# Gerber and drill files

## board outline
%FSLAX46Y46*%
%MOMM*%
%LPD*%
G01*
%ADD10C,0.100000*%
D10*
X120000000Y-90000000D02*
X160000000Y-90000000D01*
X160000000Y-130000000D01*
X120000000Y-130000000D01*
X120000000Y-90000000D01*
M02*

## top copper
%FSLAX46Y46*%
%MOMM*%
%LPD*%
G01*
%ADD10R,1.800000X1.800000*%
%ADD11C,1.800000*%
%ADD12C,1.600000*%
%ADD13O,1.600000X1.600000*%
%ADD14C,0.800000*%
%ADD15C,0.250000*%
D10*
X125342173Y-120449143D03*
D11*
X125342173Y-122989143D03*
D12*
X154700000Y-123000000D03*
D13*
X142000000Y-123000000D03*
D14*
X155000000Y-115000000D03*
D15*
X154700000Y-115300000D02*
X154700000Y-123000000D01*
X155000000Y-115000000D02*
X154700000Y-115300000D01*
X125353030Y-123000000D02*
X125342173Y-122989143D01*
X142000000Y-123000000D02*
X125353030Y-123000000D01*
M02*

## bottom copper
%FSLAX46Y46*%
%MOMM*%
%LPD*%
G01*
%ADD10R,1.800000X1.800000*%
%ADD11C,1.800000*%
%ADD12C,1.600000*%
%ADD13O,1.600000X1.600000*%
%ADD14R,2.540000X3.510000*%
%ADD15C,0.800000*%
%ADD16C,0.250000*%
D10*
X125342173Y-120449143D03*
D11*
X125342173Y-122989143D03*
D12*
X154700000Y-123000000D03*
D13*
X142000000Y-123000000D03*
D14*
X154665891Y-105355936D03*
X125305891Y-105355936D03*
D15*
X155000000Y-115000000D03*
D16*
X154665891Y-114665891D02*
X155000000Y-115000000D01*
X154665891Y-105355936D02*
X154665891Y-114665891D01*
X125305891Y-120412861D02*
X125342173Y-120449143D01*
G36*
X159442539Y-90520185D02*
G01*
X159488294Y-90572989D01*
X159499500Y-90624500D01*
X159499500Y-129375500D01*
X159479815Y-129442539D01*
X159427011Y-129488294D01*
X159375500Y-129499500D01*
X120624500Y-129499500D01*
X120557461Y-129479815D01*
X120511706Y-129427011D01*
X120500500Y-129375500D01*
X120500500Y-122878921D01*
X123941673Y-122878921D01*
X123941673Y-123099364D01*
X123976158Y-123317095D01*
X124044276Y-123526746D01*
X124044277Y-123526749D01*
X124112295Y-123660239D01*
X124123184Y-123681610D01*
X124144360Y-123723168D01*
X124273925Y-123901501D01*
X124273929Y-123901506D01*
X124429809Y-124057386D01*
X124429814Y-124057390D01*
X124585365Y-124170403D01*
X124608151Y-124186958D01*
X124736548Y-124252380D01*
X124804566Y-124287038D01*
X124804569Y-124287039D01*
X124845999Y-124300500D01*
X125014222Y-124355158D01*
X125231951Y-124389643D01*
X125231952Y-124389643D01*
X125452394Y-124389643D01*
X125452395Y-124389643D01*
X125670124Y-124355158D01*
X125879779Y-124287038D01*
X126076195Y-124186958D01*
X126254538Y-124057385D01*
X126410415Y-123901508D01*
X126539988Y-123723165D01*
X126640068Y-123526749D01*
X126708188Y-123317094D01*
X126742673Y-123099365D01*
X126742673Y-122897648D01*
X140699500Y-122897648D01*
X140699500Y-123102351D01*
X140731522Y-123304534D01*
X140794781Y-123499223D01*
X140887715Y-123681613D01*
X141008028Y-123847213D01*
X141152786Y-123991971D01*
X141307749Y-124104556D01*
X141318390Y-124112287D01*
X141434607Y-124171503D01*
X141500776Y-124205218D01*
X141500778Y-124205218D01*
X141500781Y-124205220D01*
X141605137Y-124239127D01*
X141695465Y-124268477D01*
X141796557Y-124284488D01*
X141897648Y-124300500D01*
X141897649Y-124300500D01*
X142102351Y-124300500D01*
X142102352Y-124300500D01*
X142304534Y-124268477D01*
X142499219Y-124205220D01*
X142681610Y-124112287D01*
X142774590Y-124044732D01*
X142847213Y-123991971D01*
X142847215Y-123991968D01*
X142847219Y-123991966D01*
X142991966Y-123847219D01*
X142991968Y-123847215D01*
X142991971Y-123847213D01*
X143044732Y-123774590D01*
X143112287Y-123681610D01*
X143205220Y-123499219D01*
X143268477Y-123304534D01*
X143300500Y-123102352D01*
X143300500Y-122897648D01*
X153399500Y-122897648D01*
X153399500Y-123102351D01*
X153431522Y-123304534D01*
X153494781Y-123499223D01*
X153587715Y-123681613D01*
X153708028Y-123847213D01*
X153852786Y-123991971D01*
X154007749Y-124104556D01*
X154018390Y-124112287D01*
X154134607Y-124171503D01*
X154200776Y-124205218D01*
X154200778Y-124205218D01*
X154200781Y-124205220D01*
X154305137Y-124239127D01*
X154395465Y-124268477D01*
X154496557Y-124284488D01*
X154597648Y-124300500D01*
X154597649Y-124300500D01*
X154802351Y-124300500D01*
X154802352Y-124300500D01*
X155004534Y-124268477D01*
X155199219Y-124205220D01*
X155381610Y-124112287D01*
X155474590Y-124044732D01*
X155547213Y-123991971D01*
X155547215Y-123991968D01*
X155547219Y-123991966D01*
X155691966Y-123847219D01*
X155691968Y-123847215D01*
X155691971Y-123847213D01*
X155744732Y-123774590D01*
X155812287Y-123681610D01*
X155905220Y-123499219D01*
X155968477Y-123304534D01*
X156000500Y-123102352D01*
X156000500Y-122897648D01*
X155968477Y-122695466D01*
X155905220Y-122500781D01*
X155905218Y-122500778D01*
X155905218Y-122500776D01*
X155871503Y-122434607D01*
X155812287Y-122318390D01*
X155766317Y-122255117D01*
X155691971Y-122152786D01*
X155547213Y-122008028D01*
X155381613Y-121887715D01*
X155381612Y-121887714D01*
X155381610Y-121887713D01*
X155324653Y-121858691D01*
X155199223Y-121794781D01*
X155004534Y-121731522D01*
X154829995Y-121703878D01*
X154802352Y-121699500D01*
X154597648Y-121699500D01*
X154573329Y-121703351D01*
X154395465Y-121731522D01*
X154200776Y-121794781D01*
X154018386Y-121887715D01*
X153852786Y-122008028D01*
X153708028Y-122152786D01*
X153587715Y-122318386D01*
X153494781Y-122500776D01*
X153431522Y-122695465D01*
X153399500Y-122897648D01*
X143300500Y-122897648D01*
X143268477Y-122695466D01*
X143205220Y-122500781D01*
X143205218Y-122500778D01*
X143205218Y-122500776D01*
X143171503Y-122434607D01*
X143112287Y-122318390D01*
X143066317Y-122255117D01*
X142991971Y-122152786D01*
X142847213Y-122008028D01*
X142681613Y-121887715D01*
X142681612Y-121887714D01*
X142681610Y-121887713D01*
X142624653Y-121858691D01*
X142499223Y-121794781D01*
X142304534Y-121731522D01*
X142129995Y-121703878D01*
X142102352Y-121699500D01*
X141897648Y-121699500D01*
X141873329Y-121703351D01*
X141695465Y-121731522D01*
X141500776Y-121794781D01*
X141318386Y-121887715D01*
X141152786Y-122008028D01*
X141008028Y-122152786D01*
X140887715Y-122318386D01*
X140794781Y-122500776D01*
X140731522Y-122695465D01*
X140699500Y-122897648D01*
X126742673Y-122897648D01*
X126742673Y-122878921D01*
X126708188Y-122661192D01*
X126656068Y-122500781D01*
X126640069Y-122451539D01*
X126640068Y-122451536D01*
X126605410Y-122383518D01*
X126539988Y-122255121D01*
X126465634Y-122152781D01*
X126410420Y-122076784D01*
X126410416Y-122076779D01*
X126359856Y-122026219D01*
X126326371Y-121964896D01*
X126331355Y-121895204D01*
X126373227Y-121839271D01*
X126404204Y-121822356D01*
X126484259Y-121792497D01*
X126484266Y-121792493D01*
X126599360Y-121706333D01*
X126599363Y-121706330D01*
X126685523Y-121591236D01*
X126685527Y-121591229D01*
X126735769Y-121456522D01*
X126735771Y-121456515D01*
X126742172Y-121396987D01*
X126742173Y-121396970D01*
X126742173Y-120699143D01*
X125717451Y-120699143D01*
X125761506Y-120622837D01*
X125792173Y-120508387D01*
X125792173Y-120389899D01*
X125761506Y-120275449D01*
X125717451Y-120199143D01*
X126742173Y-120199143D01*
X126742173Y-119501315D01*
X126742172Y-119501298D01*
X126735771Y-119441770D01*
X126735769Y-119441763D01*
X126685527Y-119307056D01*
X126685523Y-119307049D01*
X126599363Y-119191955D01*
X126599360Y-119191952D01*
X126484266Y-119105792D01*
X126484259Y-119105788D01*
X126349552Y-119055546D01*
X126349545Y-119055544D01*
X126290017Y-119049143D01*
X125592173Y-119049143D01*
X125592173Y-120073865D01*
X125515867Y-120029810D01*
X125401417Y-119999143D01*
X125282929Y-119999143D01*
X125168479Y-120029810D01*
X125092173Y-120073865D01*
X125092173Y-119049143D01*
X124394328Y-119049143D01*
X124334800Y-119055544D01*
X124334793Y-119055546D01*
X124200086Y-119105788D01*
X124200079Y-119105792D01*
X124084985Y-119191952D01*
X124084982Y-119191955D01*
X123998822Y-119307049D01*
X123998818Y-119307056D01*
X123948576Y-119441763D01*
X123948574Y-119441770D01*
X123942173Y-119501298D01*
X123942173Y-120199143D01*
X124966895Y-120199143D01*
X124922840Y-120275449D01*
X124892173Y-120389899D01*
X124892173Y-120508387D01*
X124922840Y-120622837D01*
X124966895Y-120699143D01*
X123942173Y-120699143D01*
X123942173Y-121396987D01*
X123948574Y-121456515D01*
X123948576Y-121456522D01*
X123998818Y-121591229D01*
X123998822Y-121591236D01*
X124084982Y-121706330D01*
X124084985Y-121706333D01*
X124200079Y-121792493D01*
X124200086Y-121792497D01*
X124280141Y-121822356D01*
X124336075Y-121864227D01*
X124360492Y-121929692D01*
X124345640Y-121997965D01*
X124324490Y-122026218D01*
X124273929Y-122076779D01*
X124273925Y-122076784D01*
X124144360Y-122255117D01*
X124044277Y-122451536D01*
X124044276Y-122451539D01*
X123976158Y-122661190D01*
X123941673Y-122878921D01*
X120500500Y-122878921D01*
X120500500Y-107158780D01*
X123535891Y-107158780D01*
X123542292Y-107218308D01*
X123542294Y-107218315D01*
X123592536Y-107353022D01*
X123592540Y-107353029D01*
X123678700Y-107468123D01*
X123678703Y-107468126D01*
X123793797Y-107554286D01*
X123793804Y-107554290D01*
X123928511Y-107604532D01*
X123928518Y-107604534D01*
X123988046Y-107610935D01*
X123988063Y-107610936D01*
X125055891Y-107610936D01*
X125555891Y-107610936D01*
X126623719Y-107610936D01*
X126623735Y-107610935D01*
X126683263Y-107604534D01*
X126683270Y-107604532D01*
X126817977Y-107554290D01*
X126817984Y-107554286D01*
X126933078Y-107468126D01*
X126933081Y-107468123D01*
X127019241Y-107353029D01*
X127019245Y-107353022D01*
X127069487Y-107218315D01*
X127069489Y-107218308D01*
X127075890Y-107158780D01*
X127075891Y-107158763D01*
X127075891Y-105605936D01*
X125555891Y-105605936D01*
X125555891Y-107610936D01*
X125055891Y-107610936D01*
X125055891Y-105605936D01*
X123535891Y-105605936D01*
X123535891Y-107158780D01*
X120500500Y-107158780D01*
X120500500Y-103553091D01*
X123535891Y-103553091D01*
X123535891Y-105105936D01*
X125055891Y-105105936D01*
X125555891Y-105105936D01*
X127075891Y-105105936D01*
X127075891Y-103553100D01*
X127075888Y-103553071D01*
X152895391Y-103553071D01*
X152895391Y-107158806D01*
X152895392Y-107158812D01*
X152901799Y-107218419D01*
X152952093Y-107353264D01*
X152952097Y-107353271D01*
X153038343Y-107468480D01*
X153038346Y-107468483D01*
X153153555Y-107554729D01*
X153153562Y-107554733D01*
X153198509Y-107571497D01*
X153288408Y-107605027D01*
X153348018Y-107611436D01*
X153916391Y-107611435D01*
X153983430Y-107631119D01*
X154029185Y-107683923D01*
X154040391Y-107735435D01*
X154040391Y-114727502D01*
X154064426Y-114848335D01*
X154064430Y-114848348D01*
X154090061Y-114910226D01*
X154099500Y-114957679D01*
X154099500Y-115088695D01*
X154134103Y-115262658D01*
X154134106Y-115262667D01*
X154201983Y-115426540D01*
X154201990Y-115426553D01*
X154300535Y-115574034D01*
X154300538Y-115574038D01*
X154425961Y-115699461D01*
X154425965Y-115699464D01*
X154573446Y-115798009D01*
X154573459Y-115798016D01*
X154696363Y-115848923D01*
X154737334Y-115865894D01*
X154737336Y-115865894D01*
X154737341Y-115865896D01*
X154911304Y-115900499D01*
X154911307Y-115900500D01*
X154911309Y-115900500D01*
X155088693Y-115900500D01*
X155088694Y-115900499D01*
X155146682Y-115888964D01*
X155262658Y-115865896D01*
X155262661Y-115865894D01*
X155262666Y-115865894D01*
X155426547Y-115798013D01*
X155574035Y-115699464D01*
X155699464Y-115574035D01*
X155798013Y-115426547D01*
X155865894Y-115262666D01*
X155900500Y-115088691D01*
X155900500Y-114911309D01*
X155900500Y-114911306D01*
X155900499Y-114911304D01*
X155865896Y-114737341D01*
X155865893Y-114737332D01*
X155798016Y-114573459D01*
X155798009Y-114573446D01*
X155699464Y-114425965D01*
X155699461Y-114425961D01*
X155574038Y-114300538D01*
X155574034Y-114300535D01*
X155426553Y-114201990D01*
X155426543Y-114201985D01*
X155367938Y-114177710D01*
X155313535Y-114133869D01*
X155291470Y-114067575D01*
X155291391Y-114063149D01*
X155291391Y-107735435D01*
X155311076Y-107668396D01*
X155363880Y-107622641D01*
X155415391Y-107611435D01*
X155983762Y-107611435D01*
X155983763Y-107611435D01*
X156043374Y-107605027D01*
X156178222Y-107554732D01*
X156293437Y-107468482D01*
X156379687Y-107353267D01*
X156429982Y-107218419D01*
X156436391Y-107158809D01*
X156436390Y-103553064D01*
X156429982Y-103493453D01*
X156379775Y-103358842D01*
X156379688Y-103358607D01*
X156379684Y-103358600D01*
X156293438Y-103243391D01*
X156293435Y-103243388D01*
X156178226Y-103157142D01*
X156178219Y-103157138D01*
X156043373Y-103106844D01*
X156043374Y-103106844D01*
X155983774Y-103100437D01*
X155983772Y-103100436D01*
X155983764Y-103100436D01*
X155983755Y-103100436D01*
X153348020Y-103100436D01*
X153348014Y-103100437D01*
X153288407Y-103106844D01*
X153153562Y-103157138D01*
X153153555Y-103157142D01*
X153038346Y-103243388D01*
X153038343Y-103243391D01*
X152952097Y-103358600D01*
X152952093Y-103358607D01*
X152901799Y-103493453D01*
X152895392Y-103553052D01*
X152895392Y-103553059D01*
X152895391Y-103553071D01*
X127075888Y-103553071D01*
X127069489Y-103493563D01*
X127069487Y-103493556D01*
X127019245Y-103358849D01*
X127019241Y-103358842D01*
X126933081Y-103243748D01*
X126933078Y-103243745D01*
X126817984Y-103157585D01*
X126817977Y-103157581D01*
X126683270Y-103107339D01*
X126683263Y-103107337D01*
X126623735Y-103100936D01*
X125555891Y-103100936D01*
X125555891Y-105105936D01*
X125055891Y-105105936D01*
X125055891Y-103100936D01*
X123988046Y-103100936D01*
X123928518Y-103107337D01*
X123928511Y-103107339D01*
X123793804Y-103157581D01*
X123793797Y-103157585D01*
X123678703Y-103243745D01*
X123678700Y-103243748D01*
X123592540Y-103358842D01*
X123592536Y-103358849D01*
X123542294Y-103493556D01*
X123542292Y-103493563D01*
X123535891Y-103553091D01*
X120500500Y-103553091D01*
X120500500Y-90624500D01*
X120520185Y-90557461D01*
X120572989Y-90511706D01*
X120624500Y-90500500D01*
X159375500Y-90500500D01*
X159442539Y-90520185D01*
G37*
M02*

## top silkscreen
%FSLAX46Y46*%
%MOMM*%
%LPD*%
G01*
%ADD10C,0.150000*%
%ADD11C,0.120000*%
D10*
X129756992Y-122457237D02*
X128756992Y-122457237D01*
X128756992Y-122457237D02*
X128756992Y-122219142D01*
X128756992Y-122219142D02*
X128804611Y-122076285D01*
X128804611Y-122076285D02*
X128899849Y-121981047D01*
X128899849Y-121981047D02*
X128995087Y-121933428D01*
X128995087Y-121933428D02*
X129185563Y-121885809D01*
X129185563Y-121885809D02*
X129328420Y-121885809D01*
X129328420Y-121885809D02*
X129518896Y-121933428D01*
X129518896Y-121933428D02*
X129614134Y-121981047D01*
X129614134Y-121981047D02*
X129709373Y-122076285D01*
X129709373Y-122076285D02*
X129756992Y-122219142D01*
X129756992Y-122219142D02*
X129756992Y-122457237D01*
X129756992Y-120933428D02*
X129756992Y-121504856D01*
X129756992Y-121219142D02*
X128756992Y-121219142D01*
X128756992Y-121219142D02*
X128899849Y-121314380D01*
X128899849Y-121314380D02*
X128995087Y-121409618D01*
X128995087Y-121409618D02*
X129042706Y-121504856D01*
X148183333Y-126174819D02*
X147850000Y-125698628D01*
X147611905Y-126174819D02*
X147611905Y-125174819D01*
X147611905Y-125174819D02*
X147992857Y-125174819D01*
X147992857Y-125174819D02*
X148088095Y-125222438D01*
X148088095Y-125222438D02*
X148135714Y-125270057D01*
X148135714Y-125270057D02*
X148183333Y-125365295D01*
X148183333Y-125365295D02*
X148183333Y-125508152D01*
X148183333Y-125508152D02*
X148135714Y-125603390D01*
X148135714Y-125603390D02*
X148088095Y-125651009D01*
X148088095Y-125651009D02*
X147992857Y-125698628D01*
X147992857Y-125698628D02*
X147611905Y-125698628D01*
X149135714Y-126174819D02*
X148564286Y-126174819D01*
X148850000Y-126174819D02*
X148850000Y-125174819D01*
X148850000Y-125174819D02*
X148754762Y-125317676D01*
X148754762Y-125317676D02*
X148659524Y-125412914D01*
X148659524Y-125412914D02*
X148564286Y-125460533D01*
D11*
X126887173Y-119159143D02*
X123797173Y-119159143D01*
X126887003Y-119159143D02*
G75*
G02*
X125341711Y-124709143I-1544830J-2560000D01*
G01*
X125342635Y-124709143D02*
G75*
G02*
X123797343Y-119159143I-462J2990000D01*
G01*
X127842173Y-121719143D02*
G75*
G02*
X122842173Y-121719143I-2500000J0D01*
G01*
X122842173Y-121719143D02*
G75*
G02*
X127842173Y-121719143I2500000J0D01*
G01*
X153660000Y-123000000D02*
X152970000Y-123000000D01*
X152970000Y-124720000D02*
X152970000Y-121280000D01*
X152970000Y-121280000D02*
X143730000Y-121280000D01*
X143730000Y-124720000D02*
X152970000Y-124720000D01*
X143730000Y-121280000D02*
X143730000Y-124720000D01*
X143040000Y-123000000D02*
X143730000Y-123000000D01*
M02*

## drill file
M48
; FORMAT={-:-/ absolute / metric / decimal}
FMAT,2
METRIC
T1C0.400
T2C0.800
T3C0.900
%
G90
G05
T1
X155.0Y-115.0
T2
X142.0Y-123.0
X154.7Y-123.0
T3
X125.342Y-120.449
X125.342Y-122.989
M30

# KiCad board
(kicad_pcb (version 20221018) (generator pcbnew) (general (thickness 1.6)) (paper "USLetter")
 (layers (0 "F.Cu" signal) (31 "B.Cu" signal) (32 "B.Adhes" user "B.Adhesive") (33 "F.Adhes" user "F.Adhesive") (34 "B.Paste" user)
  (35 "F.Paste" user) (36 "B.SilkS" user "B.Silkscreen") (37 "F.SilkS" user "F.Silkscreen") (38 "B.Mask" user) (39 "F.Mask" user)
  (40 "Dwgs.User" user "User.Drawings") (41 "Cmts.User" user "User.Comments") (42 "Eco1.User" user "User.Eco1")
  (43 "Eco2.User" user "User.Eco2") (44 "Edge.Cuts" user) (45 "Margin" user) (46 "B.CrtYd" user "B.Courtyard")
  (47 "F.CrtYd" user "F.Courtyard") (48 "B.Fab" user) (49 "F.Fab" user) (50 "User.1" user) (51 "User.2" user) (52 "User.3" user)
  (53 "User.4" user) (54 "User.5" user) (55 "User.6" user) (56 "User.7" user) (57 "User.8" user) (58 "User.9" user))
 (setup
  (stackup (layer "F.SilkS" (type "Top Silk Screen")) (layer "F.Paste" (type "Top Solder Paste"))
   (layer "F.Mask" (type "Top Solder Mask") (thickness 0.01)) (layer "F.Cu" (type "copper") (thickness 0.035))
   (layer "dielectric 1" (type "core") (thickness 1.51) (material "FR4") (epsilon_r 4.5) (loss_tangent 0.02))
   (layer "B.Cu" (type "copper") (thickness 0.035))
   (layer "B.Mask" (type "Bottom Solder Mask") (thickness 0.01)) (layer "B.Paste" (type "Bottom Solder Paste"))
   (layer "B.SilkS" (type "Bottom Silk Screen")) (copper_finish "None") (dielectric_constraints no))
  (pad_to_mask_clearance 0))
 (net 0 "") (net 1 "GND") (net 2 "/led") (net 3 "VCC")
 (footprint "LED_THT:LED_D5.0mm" (layer "F.Cu") (at 125.342173 120.449143 -90)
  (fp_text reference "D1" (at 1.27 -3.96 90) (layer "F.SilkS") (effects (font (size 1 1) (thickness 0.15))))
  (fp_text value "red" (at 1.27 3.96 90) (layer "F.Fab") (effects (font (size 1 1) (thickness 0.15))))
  (fp_line (start -1.29 -1.545) (end -1.29 1.545) (stroke (width 0.12) (type solid)) (layer "F.SilkS"))
  (fp_arc (start -1.29 -1.54483) (mid 2.072002 -2.880433) (end 4.26 0.000462) (stroke (width 0.12) (type solid)) (layer "F.SilkS"))
  (fp_arc (start 4.26 -0.000462) (mid 2.072002 2.880433) (end -1.29 1.54483) (stroke (width 0.12) (type solid)) (layer "F.SilkS"))
  (fp_circle (center 1.27 0) (end 3.77 0) (stroke (width 0.12) (type solid)) (fill none) (layer "F.SilkS"))
  (pad "1" thru_hole rect (at 0 0 270) (size 1.8 1.8) (drill 0.9) (layers "*.Cu" "*.Mask") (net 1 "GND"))
  (pad "2" thru_hole circle (at 2.54 0 270) (size 1.8 1.8) (drill 0.9) (layers "*.Cu" "*.Mask") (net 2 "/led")))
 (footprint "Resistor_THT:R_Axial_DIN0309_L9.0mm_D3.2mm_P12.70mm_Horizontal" (layer "F.Cu") (at 154.7 123 180)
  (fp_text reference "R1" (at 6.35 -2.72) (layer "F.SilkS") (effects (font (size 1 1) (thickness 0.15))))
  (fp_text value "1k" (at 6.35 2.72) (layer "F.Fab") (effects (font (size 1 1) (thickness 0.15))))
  (fp_line (start 1.04 0) (end 1.73 0) (stroke (width 0.12) (type solid)) (layer "F.SilkS"))
  (fp_line (start 1.73 -1.72) (end 1.73 1.72) (stroke (width 0.12) (type solid)) (layer "F.SilkS"))
  (fp_line (start 1.73 1.72) (end 10.97 1.72) (stroke (width 0.12) (type solid)) (layer "F.SilkS"))
  (fp_line (start 10.97 -1.72) (end 1.73 -1.72) (stroke (width 0.12) (type solid)) (layer "F.SilkS"))
  (fp_line (start 10.97 1.72) (end 10.97 -1.72) (stroke (width 0.12) (type solid)) (layer "F.SilkS"))
  (fp_line (start 11.66 0) (end 10.97 0) (stroke (width 0.12) (type solid)) (layer "F.SilkS"))
  (pad "1" thru_hole circle (at 0 0 180) (size 1.6 1.6) (drill 0.8) (layers "*.Cu" "*.Mask") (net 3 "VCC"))
  (pad "2" thru_hole oval (at 12.7 0 180) (size 1.6 1.6) (drill 0.8) (layers "*.Cu" "*.Mask") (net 2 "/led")))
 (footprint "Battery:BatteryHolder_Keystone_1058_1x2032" (layer "B.Cu") (at 139.985891 105.355936 180)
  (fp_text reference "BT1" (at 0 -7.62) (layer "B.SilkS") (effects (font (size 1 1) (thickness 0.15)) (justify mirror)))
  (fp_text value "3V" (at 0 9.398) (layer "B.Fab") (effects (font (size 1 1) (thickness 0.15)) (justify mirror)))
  (pad "1" smd rect (at -14.68 0 180) (size 2.54 3.51) (layers "B.Cu" "B.Paste" "B.Mask") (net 3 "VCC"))
  (pad "2" smd rect (at 14.68 0 180) (size 2.54 3.51) (layers "B.Cu" "B.Paste" "B.Mask") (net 1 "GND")))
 (gr_rect (start 120 90) (end 160 130) (stroke (width 0.1) (type default)) (fill none) (layer "Edge.Cuts"))
 (segment (start 154.7 115.3) (end 154.7 123) (width 0.25) (layer "F.Cu") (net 3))
 (segment (start 155 115) (end 154.7 115.3) (width 0.25) (layer "F.Cu") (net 3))
 (via (at 155 115) (size 0.8) (drill 0.4) (layers "F.Cu" "B.Cu") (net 3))
 (segment (start 154.665891 114.665891) (end 155 115) (width 0.25) (layer "B.Cu") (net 3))
 (segment (start 154.665891 105.355936) (end 154.665891 114.665891) (width 0.25) (layer "B.Cu") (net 3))
 (segment (start 125.305891 120.412861) (end 125.342173 120.449143) (width 0.25) (layer "B.Cu") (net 1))
 (segment (start 125.35303 123) (end 125.342173 122.989143) (width 0.25) (layer "F.Cu") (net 2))
 (segment (start 142 123) (end 125.35303 123) (width 0.25) (layer "F.Cu") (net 2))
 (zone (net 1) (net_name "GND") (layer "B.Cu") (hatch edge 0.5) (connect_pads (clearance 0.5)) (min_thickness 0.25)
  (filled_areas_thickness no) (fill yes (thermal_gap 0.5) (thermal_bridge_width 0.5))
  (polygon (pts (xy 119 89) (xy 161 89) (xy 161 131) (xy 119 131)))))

